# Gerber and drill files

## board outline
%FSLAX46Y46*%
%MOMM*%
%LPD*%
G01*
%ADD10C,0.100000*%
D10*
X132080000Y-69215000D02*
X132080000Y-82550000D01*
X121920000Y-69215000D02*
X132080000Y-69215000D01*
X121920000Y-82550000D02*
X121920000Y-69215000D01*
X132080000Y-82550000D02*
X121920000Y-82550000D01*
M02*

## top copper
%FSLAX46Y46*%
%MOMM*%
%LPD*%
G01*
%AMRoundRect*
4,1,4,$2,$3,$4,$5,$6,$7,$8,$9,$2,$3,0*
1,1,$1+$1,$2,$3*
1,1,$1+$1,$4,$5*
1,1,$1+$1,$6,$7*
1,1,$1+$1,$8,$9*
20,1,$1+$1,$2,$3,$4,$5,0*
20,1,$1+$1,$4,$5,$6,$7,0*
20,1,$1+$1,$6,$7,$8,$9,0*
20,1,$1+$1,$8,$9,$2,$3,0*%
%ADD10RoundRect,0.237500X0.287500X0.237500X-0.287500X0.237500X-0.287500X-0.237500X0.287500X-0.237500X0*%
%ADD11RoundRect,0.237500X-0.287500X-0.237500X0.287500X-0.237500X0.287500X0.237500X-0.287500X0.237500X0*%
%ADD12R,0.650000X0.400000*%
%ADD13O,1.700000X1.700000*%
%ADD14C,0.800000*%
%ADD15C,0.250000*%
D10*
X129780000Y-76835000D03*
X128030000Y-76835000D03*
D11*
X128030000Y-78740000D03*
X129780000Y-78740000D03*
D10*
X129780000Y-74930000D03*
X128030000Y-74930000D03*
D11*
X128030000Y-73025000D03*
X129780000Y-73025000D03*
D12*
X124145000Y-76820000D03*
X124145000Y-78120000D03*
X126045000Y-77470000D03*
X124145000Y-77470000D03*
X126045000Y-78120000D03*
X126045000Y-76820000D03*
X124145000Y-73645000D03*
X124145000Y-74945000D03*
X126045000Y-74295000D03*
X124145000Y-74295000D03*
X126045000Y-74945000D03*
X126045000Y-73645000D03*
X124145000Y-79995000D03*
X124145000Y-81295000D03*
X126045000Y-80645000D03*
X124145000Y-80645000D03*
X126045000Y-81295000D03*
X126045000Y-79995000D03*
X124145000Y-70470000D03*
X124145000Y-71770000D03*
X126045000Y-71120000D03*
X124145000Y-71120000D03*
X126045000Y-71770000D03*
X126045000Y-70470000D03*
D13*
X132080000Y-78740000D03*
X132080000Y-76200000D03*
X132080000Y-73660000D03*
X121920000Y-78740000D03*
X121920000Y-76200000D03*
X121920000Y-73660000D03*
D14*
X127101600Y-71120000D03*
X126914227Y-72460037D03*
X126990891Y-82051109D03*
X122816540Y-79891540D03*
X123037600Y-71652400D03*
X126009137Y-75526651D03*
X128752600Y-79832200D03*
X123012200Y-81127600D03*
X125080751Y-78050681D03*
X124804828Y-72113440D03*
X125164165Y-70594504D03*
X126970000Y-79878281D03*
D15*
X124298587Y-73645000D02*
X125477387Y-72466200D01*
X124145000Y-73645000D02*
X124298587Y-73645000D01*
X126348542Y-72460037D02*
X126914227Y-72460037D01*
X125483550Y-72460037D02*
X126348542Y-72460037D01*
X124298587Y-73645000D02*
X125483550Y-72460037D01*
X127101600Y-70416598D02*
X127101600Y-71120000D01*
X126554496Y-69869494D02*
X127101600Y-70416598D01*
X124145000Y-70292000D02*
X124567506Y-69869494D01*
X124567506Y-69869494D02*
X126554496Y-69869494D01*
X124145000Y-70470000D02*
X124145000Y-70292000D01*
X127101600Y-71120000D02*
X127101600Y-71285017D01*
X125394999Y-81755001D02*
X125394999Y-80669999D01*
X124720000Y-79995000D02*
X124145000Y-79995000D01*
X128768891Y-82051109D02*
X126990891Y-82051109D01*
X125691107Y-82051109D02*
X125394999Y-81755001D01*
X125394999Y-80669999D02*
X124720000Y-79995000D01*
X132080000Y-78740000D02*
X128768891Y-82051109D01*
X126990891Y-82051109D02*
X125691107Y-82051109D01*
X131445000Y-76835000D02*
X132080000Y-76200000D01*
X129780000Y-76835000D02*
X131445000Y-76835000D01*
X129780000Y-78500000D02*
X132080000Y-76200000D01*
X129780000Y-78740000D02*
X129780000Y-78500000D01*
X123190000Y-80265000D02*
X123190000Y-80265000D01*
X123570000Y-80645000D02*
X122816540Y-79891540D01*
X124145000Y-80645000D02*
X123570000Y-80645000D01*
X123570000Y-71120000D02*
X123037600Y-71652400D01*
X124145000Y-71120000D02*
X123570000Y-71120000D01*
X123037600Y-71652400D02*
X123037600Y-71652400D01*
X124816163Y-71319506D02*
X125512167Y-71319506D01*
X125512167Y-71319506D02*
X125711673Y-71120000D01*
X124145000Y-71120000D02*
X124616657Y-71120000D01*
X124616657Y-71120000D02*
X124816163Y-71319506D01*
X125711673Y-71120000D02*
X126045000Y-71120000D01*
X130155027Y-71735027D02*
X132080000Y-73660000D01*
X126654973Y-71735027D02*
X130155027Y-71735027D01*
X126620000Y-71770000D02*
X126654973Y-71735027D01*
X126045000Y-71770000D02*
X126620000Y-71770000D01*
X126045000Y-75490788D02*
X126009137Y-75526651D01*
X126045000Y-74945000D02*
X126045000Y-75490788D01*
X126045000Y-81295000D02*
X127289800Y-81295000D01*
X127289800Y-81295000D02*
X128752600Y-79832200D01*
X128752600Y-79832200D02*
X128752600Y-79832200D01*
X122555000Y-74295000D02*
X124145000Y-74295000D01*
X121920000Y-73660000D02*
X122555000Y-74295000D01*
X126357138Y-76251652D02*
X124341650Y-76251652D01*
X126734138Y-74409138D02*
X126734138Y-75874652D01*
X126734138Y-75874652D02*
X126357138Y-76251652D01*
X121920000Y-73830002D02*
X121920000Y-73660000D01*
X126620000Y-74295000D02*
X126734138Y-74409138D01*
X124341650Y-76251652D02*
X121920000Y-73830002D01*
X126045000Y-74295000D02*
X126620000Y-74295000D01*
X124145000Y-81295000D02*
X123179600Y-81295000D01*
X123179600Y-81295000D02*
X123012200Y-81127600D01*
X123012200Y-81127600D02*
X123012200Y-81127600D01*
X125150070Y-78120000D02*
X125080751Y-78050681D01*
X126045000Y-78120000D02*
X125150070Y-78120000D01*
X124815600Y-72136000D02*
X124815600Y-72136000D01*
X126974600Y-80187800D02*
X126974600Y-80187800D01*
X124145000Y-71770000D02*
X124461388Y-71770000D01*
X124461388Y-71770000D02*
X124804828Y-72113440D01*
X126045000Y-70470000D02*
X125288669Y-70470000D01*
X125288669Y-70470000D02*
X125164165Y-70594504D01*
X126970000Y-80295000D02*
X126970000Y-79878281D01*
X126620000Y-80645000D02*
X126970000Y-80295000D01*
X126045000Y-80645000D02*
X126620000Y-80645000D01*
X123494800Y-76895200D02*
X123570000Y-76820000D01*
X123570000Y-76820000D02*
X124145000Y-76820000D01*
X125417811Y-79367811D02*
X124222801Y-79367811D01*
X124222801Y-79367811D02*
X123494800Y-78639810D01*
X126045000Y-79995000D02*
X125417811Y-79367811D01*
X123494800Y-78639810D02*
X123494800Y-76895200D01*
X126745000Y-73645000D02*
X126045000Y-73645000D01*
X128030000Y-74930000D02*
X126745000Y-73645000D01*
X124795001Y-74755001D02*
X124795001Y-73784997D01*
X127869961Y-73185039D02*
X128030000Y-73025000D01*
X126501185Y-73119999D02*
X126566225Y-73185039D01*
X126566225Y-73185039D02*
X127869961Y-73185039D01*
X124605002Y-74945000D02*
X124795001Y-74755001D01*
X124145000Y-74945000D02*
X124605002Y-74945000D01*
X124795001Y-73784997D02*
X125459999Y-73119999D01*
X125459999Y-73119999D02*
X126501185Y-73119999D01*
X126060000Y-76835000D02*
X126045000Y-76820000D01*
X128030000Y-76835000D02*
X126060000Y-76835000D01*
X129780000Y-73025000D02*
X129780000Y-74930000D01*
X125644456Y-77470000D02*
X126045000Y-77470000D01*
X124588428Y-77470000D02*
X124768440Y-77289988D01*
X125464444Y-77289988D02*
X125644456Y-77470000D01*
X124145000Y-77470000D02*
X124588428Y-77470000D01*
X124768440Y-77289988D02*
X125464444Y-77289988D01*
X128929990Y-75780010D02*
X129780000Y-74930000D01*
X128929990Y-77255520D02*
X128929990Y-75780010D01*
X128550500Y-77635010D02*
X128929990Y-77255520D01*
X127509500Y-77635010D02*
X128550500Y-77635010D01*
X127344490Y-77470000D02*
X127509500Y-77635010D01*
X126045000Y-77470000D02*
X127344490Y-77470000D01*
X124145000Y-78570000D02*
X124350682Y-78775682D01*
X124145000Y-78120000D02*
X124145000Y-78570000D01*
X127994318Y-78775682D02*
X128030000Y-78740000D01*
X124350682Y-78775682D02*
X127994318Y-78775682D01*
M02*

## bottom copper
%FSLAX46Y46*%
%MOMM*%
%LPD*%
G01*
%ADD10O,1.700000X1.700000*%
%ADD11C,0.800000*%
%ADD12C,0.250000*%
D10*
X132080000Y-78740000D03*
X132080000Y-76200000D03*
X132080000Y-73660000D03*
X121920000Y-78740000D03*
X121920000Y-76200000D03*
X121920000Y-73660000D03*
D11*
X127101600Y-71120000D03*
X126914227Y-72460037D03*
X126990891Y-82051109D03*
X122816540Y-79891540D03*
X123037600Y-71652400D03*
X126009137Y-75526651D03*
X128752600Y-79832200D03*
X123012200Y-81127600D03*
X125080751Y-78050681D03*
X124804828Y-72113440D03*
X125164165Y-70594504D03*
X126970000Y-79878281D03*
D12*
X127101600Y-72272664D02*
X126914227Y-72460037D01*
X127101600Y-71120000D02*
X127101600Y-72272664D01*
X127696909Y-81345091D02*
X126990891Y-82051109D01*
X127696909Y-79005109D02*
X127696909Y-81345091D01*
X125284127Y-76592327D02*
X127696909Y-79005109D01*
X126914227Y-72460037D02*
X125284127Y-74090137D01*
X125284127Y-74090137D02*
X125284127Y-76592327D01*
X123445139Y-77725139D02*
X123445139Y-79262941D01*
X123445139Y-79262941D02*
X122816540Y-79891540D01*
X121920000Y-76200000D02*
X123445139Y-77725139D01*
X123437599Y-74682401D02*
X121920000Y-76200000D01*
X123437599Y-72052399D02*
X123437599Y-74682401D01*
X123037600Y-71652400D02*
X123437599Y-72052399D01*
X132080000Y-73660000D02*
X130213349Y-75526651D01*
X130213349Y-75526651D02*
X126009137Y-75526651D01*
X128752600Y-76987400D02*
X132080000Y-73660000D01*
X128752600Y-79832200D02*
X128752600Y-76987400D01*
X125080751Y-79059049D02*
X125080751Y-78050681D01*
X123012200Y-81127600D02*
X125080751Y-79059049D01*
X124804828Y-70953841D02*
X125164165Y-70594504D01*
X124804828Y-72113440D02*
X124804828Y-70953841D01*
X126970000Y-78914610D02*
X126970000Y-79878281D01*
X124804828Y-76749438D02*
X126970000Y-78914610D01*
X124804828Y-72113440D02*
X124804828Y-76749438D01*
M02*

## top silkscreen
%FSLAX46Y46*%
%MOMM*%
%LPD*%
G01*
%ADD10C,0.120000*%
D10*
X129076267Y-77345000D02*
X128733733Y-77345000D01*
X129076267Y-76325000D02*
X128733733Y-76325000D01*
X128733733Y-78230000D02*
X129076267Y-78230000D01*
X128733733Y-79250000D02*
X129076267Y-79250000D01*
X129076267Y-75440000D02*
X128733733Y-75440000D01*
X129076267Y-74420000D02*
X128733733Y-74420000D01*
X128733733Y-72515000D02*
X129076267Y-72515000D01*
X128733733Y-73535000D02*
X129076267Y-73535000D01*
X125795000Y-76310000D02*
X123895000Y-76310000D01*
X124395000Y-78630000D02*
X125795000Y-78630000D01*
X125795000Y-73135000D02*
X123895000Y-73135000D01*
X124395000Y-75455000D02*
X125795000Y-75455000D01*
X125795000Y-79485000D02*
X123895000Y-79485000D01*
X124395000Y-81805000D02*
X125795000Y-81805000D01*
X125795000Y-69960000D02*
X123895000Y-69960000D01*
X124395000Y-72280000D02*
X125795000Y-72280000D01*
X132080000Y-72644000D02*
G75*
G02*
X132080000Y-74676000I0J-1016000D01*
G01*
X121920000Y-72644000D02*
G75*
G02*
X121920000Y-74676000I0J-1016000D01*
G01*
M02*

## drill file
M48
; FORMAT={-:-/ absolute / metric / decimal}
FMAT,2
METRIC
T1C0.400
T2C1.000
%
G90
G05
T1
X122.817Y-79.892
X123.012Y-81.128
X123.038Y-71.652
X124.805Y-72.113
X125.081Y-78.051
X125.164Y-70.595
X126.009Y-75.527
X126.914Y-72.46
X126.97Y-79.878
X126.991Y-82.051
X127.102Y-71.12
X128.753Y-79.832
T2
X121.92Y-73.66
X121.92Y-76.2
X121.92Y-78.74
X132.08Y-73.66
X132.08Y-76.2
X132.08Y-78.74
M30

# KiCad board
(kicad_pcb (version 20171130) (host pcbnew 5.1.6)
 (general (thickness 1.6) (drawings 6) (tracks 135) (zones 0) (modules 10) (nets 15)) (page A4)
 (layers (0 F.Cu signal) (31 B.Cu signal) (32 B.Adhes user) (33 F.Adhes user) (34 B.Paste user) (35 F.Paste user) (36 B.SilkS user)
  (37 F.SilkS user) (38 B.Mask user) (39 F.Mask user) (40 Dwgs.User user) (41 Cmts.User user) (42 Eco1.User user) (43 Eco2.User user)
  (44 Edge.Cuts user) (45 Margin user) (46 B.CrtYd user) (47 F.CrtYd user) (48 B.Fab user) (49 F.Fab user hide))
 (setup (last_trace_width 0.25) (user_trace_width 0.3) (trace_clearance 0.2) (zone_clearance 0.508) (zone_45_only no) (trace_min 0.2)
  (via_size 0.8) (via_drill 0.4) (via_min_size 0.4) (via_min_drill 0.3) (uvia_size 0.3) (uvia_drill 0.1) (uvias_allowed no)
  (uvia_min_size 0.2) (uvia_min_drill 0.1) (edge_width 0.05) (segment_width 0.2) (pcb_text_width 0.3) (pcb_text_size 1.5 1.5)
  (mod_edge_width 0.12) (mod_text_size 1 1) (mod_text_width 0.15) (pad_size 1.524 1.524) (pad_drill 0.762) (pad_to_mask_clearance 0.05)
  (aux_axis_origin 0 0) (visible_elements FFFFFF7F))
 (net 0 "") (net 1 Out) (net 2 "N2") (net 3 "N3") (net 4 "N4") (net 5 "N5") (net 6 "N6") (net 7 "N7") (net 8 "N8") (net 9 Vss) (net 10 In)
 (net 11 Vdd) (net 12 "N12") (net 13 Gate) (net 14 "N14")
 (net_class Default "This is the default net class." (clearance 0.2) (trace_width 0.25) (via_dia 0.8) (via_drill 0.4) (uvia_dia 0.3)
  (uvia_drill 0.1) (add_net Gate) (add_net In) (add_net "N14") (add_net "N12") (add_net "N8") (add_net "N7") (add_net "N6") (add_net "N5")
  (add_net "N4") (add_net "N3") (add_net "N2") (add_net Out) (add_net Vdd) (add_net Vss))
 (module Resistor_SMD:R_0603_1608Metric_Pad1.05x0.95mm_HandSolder (layer F.Cu) (at 128.905 76.835 180)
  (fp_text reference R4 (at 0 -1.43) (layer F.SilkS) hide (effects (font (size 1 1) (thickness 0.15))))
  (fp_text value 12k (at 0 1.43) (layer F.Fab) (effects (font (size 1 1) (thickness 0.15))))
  (fp_line (start -0.171267 -0.51) (end 0.171267 -0.51) (layer F.SilkS) (width 0.12))
  (fp_line (start -0.171267 0.51) (end 0.171267 0.51) (layer F.SilkS) (width 0.12))
  (pad 1 smd roundrect (at -0.875 0 180) (size 1.05 0.95) (layers F.Cu F.Paste F.Mask) (roundrect_rratio 0.25) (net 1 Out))
  (pad 2 smd roundrect (at 0.875 0 180) (size 1.05 0.95) (layers F.Cu F.Paste F.Mask) (roundrect_rratio 0.25) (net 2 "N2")))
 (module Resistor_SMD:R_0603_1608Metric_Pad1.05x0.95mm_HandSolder (layer F.Cu) (at 128.905 78.74)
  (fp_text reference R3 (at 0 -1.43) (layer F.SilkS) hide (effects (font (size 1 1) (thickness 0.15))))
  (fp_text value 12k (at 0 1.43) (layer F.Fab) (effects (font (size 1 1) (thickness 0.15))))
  (fp_line (start -0.171267 -0.51) (end 0.171267 -0.51) (layer F.SilkS) (width 0.12))
  (fp_line (start -0.171267 0.51) (end 0.171267 0.51) (layer F.SilkS) (width 0.12))
  (pad 1 smd roundrect (at -0.875 0) (size 1.05 0.95) (layers F.Cu F.Paste F.Mask) (roundrect_rratio 0.25) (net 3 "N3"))
  (pad 2 smd roundrect (at 0.875 0) (size 1.05 0.95) (layers F.Cu F.Paste F.Mask) (roundrect_rratio 0.25) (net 1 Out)))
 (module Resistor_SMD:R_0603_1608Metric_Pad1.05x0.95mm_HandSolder (layer F.Cu) (at 128.905 74.93 180)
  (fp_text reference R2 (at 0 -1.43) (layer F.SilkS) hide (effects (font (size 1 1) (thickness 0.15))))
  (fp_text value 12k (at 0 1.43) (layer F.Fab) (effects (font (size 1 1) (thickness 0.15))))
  (fp_line (start -0.171267 -0.51) (end 0.171267 -0.51) (layer F.SilkS) (width 0.12))
  (fp_line (start -0.171267 0.51) (end 0.171267 0.51) (layer F.SilkS) (width 0.12))
  (pad 1 smd roundrect (at -0.875 0 180) (size 1.05 0.95) (layers F.Cu F.Paste F.Mask) (roundrect_rratio 0.25) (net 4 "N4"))
  (pad 2 smd roundrect (at 0.875 0 180) (size 1.05 0.95) (layers F.Cu F.Paste F.Mask) (roundrect_rratio 0.25) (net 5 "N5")))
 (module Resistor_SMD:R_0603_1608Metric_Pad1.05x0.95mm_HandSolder (layer F.Cu) (at 128.905 73.025)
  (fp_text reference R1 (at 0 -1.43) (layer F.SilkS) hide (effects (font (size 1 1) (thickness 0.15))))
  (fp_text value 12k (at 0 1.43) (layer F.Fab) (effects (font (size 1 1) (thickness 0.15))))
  (fp_line (start -0.171267 -0.51) (end 0.171267 -0.51) (layer F.SilkS) (width 0.12))
  (fp_line (start -0.171267 0.51) (end 0.171267 0.51) (layer F.SilkS) (width 0.12))
  (pad 1 smd roundrect (at -0.875 0) (size 1.05 0.95) (layers F.Cu F.Paste F.Mask) (roundrect_rratio 0.25) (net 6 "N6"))
  (pad 2 smd roundrect (at 0.875 0) (size 1.05 0.95) (layers F.Cu F.Paste F.Mask) (roundrect_rratio 0.25) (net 4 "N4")))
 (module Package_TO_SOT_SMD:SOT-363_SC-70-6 (layer F.Cu) (at 125.095 77.47)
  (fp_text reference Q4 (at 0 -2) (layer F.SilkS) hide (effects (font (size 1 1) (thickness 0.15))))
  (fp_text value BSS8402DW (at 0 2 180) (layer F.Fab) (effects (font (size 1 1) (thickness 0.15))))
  (fp_line (start 0.7 -1.16) (end -1.2 -1.16) (layer F.SilkS) (width 0.12))
  (fp_line (start -0.7 1.16) (end 0.7 1.16) (layer F.SilkS) (width 0.12))
  (pad 1 smd rect (at -0.95 -0.65) (size 0.65 0.4) (layers F.Cu F.Paste F.Mask) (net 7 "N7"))
  (pad 3 smd rect (at -0.95 0.65) (size 0.65 0.4) (layers F.Cu F.Paste F.Mask) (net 3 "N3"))
  (pad 5 smd rect (at 0.95 0) (size 0.65 0.4) (layers F.Cu F.Paste F.Mask) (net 4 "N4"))
  (pad 2 smd rect (at -0.95 0) (size 0.65 0.4) (layers F.Cu F.Paste F.Mask) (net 4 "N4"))
  (pad 4 smd rect (at 0.95 0.65) (size 0.65 0.4) (layers F.Cu F.Paste F.Mask) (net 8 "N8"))
  (pad 6 smd rect (at 0.95 -0.65) (size 0.65 0.4) (layers F.Cu F.Paste F.Mask) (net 2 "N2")))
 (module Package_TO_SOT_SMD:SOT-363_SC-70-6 (layer F.Cu) (at 125.095 74.295)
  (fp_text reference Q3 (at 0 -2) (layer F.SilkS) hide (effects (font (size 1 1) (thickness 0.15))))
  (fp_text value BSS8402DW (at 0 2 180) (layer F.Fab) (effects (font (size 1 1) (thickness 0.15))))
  (fp_line (start 0.7 -1.16) (end -1.2 -1.16) (layer F.SilkS) (width 0.12))
  (fp_line (start -0.7 1.16) (end 0.7 1.16) (layer F.SilkS) (width 0.12))
  (pad 1 smd rect (at -0.95 -0.65) (size 0.65 0.4) (layers F.Cu F.Paste F.Mask) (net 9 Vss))
  (pad 3 smd rect (at -0.95 0.65) (size 0.65 0.4) (layers F.Cu F.Paste F.Mask) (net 6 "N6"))
  (pad 5 smd rect (at 0.95 0) (size 0.65 0.4) (layers F.Cu F.Paste F.Mask) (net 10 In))
  (pad 2 smd rect (at -0.95 0) (size 0.65 0.4) (layers F.Cu F.Paste F.Mask) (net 10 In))
  (pad 4 smd rect (at 0.95 0.65) (size 0.65 0.4) (layers F.Cu F.Paste F.Mask) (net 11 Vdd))
  (pad 6 smd rect (at 0.95 -0.65) (size 0.65 0.4) (layers F.Cu F.Paste F.Mask) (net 5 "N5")))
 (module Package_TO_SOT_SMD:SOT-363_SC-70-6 (layer F.Cu) (at 125.095 80.645)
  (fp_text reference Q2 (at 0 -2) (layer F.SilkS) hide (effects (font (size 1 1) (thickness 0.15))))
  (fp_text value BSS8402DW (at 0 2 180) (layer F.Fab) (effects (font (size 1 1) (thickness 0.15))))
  (fp_line (start 0.7 -1.16) (end -1.2 -1.16) (layer F.SilkS) (width 0.12))
  (fp_line (start -0.7 1.16) (end 0.7 1.16) (layer F.SilkS) (width 0.12))
  (pad 1 smd rect (at -0.95 -0.65) (size 0.65 0.4) (layers F.Cu F.Paste F.Mask) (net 9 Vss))
  (pad 3 smd rect (at -0.95 0.65) (size 0.65 0.4) (layers F.Cu F.Paste F.Mask) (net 8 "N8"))
  (pad 5 smd rect (at 0.95 0) (size 0.65 0.4) (layers F.Cu F.Paste F.Mask) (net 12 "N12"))
  (pad 2 smd rect (at -0.95 0) (size 0.65 0.4) (layers F.Cu F.Paste F.Mask) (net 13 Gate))
  (pad 4 smd rect (at 0.95 0.65) (size 0.65 0.4) (layers F.Cu F.Paste F.Mask) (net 11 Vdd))
  (pad 6 smd rect (at 0.95 -0.65) (size 0.65 0.4) (layers F.Cu F.Paste F.Mask) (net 7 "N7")))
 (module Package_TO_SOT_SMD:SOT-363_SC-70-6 (layer F.Cu) (at 125.095 71.12)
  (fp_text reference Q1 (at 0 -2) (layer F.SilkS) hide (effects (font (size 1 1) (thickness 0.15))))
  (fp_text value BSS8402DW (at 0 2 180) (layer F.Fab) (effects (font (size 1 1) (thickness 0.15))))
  (fp_line (start 0.7 -1.16) (end -1.2 -1.16) (layer F.SilkS) (width 0.12))
  (fp_line (start -0.7 1.16) (end 0.7 1.16) (layer F.SilkS) (width 0.12))
  (pad 1 smd rect (at -0.95 -0.65) (size 0.65 0.4) (layers F.Cu F.Paste F.Mask) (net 9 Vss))
  (pad 3 smd rect (at -0.95 0.65) (size 0.65 0.4) (layers F.Cu F.Paste F.Mask) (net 12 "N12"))
  (pad 5 smd rect (at 0.95 0) (size 0.65 0.4) (layers F.Cu F.Paste F.Mask) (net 13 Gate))
  (pad 2 smd rect (at -0.95 0) (size 0.65 0.4) (layers F.Cu F.Paste F.Mask) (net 13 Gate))
  (pad 4 smd rect (at 0.95 0.65) (size 0.65 0.4) (layers F.Cu F.Paste F.Mask) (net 11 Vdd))
  (pad 6 smd rect (at 0.95 -0.65) (size 0.65 0.4) (layers F.Cu F.Paste F.Mask) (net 12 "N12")))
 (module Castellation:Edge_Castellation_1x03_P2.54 (layer F.Cu) (at 132.08 73.66)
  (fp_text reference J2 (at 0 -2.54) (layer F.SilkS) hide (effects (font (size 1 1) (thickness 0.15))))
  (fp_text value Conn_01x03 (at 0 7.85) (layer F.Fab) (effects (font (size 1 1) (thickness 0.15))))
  (fp_arc (start 0 0) (end 0 1.016) (angle -180) (layer F.SilkS) (width 0.12))
  (pad 3 thru_hole oval (at 0 5.08) (size 1.7 1.7) (drill 1) (layers *.Cu *.Mask) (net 9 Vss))
  (pad 2 thru_hole oval (at 0 2.54) (size 1.7 1.7) (drill 1) (layers *.Cu *.Mask) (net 1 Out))
  (pad 1 thru_hole oval (at 0 0) (size 1.7 1.7) (drill 1) (layers *.Cu *.Mask) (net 11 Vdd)))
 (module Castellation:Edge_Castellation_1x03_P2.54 (layer F.Cu) (at 121.92 73.66)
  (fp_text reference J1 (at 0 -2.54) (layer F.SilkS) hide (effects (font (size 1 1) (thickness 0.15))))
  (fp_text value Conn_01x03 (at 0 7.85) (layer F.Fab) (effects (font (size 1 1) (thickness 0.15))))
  (fp_arc (start 0 0) (end 0 1.016) (angle -180) (layer F.SilkS) (width 0.12))
  (pad 3 thru_hole oval (at 0 5.08) (size 1.7 1.7) (drill 1) (layers *.Cu *.Mask) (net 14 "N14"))
  (pad 2 thru_hole oval (at 0 2.54) (size 1.7 1.7) (drill 1) (layers *.Cu *.Mask) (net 13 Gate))
  (pad 1 thru_hole oval (at 0 0) (size 1.7 1.7) (drill 1) (layers *.Cu *.Mask) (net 10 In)))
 (gr_line (start 132.08 69.215) (end 132.08 82.55) (layer Edge.Cuts) (width 0.1))
 (gr_line (start 121.92 69.215) (end 132.08 69.215) (layer Edge.Cuts) (width 0.1))
 (gr_line (start 121.92 82.55) (end 121.92 69.215) (layer Edge.Cuts) (width 0.1))
 (gr_line (start 132.08 82.55) (end 121.92 82.55) (layer Edge.Cuts) (width 0.1))
 (via (at 127.1016 71.12) (size 0.8) (drill 0.4) (layers F.Cu B.Cu) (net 9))
 (segment (start 124.298587 73.645) (end 125.477387 72.4662) (width 0.25) (layer F.Cu) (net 9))
 (segment (start 124.145 73.645) (end 124.298587 73.645) (width 0.25) (layer F.Cu) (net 9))
 (segment (start 126.348542 72.460037) (end 126.914227 72.460037) (width 0.25) (layer F.Cu) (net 9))
 (segment (start 125.48355 72.460037) (end 126.348542 72.460037) (width 0.25) (layer F.Cu) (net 9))
 (via (at 126.914227 72.460037) (size 0.8) (drill 0.4) (layers F.Cu B.Cu) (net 9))
 (segment (start 124.298587 73.645) (end 125.48355 72.460037) (width 0.25) (layer F.Cu) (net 9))
 (segment (start 127.1016 70.416598) (end 127.1016 71.12) (width 0.25) (layer F.Cu) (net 9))
 (segment (start 126.554496 69.869494) (end 127.1016 70.416598) (width 0.25) (layer F.Cu) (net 9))
 (segment (start 124.145 70.292) (end 124.567506 69.869494) (width 0.25) (layer F.Cu) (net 9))
 (segment (start 124.567506 69.869494) (end 126.554496 69.869494) (width 0.25) (layer F.Cu) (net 9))
 (segment (start 124.145 70.47) (end 124.145 70.292) (width 0.25) (layer F.Cu) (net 9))
 (segment (start 127.1016 71.12) (end 127.1016 71.285017) (width 0.25) (layer F.Cu) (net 9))
 (segment (start 127.1016 72.272664) (end 126.914227 72.460037) (width 0.25) (layer B.Cu) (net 9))
 (segment (start 127.1016 71.12) (end 127.1016 72.272664) (width 0.25) (layer B.Cu) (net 9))
 (segment (start 125.394999 81.755001) (end 125.394999 80.669999) (width 0.25) (layer F.Cu) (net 9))
 (segment (start 124.72 79.995) (end 124.145 79.995) (width 0.25) (layer F.Cu) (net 9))
 (segment (start 128.768891 82.051109) (end 126.990891 82.051109) (width 0.25) (layer F.Cu) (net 9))
 (segment (start 125.691107 82.051109) (end 125.394999 81.755001) (width 0.25) (layer F.Cu) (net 9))
 (segment (start 125.394999 80.669999) (end 124.72 79.995) (width 0.25) (layer F.Cu) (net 9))
 (segment (start 132.08 78.74) (end 128.768891 82.051109) (width 0.25) (layer F.Cu) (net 9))
 (segment (start 126.990891 82.051109) (end 125.691107 82.051109) (width 0.25) (layer F.Cu) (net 9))
 (via (at 126.990891 82.051109) (size 0.8) (drill 0.4) (layers F.Cu B.Cu) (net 9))
 (segment (start 127.696909 81.345091) (end 126.990891 82.051109) (width 0.25) (layer B.Cu) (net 9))
 (segment (start 127.696909 79.005109) (end 127.696909 81.345091) (width 0.25) (layer B.Cu) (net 9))
 (segment (start 125.284127 76.592327) (end 127.696909 79.005109) (width 0.25) (layer B.Cu) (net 9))
 (segment (start 126.914227 72.460037) (end 125.284127 74.090137) (width 0.25) (layer B.Cu) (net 9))
 (segment (start 125.284127 74.090137) (end 125.284127 76.592327) (width 0.25) (layer B.Cu) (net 9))
 (segment (start 131.445 76.835) (end 132.08 76.2) (width 0.25) (layer F.Cu) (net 1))
 (segment (start 129.78 76.835) (end 131.445 76.835) (width 0.25) (layer F.Cu) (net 1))
 (segment (start 129.78 78.5) (end 132.08 76.2) (width 0.25) (layer F.Cu) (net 1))
 (segment (start 129.78 78.74) (end 129.78 78.5) (width 0.25) (layer F.Cu) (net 1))
 (segment (start 123.19 80.265) (end 123.19 80.265) (width 0.25) (layer F.Cu) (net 13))
 (segment (start 123.445139 77.725139) (end 123.445139 79.262941) (width 0.25) (layer B.Cu) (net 13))
 (segment (start 123.57 80.645) (end 122.81654 79.89154) (width 0.25) (layer F.Cu) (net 13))
 (segment (start 124.145 80.645) (end 123.57 80.645) (width 0.25) (layer F.Cu) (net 13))
 (segment (start 123.445139 79.262941) (end 122.81654 79.89154) (width 0.25) (layer B.Cu) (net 13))
 (via (at 122.81654 79.89154) (size 0.8) (drill 0.4) (layers F.Cu B.Cu) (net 13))
 (segment (start 121.92 76.2) (end 123.445139 77.725139) (width 0.25) (layer B.Cu) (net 13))
 (segment (start 123.57 71.12) (end 123.0376 71.6524) (width 0.25) (layer F.Cu) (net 13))
 (segment (start 124.145 71.12) (end 123.57 71.12) (width 0.25) (layer F.Cu) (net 13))
 (segment (start 123.0376 71.6524) (end 123.0376 71.6524) (width 0.25) (layer F.Cu) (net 13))
 (via (at 123.0376 71.6524) (size 0.8) (drill 0.4) (layers F.Cu B.Cu) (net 13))
 (segment (start 123.437599 74.682401) (end 121.92 76.2) (width 0.25) (layer B.Cu) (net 13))
 (segment (start 123.437599 72.052399) (end 123.437599 74.682401) (width 0.25) (layer B.Cu) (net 13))
 (segment (start 123.0376 71.6524) (end 123.437599 72.052399) (width 0.25) (layer B.Cu) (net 13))
 (segment (start 124.816163 71.319506) (end 125.512167 71.319506) (width 0.25) (layer F.Cu) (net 13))
 (segment (start 125.512167 71.319506) (end 125.711673 71.12) (width 0.25) (layer F.Cu) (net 13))
 (segment (start 124.145 71.12) (end 124.616657 71.12) (width 0.25) (layer F.Cu) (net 13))
 (segment (start 124.616657 71.12) (end 124.816163 71.319506) (width 0.25) (layer F.Cu) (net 13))
 (segment (start 125.711673 71.12) (end 126.045 71.12) (width 0.25) (layer F.Cu) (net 13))
 (segment (start 130.155027 71.735027) (end 132.08 73.66) (width 0.25) (layer F.Cu) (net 11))
 (segment (start 126.654973 71.735027) (end 130.155027 71.735027) (width 0.25) (layer F.Cu) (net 11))
 (segment (start 126.62 71.77) (end 126.654973 71.735027) (width 0.25) (layer F.Cu) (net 11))
 (segment (start 126.045 71.77) (end 126.62 71.77) (width 0.25) (layer F.Cu) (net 11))
 (via (at 126.009137 75.526651) (size 0.8) (drill 0.4) (layers F.Cu B.Cu) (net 11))
 (segment (start 132.08 73.66) (end 130.213349 75.526651) (width 0.25) (layer B.Cu) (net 11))
 (segment (start 130.213349 75.526651) (end 126.009137 75.526651) (width 0.25) (layer B.Cu) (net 11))
 (segment (start 126.045 75.490788) (end 126.009137 75.526651) (width 0.25) (layer F.Cu) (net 11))
 (segment (start 126.045 74.945) (end 126.045 75.490788) (width 0.25) (layer F.Cu) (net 11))
 (segment (start 126.045 81.295) (end 127.2898 81.295) (width 0.25) (layer F.Cu) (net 11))
 (segment (start 127.2898 81.295) (end 128.7526 79.8322) (width 0.25) (layer F.Cu) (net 11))
 (segment (start 128.7526 79.8322) (end 128.7526 79.8322) (width 0.25) (layer F.Cu) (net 11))
 (via (at 128.7526 79.8322) (size 0.8) (drill 0.4) (layers F.Cu B.Cu) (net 11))
 (segment (start 128.7526 76.9874) (end 132.08 73.66) (width 0.25) (layer B.Cu) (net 11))
 (segment (start 128.7526 79.8322) (end 128.7526 76.9874) (width 0.25) (layer B.Cu) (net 11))
 (segment (start 122.555 74.295) (end 124.145 74.295) (width 0.25) (layer F.Cu) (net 10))
 (segment (start 121.92 73.66) (end 122.555 74.295) (width 0.25) (layer F.Cu) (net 10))
 (segment (start 126.357138 76.251652) (end 124.34165 76.251652) (width 0.25) (layer F.Cu) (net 10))
 (segment (start 126.734138 74.409138) (end 126.734138 75.874652) (width 0.25) (layer F.Cu) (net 10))
 (segment (start 126.734138 75.874652) (end 126.357138 76.251652) (width 0.25) (layer F.Cu) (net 10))
 (segment (start 121.92 73.830002) (end 121.92 73.66) (width 0.25) (layer F.Cu) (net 10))
 (segment (start 126.62 74.295) (end 126.734138 74.409138) (width 0.25) (layer F.Cu) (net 10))
 (segment (start 124.34165 76.251652) (end 121.92 73.830002) (width 0.25) (layer F.Cu) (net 10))
 (segment (start 126.045 74.295) (end 126.62 74.295) (width 0.25) (layer F.Cu) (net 10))
 (segment (start 124.145 81.295) (end 123.1796 81.295) (width 0.25) (layer F.Cu) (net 8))
 (segment (start 123.1796 81.295) (end 123.0122 81.1276) (width 0.25) (layer F.Cu) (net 8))
 (segment (start 123.0122 81.1276) (end 123.0122 81.1276) (width 0.25) (layer F.Cu) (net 8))
 (via (at 123.0122 81.1276) (size 0.8) (drill 0.4) (layers F.Cu B.Cu) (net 8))
 (segment (start 125.15007 78.12) (end 125.080751 78.050681) (width 0.25) (layer F.Cu) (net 8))
 (via (at 125.080751 78.050681) (size 0.8) (drill 0.4) (layers F.Cu B.Cu) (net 8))
 (segment (start 125.080751 79.059049) (end 125.080751 78.050681) (width 0.25) (layer B.Cu) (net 8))
 (segment (start 123.0122 81.1276) (end 125.080751 79.059049) (width 0.25) (layer B.Cu) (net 8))
 (segment (start 126.045 78.12) (end 125.15007 78.12) (width 0.25) (layer F.Cu) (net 8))
 (segment (start 124.8156 72.136) (end 124.8156 72.136) (width 0.25) (layer F.Cu) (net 12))
 (segment (start 126.9746 80.1878) (end 126.9746 80.1878) (width 0.25) (layer F.Cu) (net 12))
 (via (at 124.804828 72.11344) (size 0.8) (drill 0.4) (layers F.Cu B.Cu) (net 12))
 (segment (start 124.145 71.77) (end 124.461388 71.77) (width 0.25) (layer F.Cu) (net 12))
 (segment (start 124.461388 71.77) (end 124.804828 72.11344) (width 0.25) (layer F.Cu) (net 12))
 (segment (start 126.045 70.47) (end 125.288669 70.47) (width 0.25) (layer F.Cu) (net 12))
 (segment (start 124.804828 70.953841) (end 125.164165 70.594504) (width 0.25) (layer B.Cu) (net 12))
 (segment (start 124.804828 72.11344) (end 124.804828 70.953841) (width 0.25) (layer B.Cu) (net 12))
 (segment (start 125.288669 70.47) (end 125.164165 70.594504) (width 0.25) (layer F.Cu) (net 12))
 (via (at 125.164165 70.594504) (size 0.8) (drill 0.4) (layers F.Cu B.Cu) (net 12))
 (segment (start 126.97 78.91461) (end 126.97 79.878281) (width 0.25) (layer B.Cu) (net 12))
 (via (at 126.97 79.878281) (size 0.8) (drill 0.4) (layers F.Cu B.Cu) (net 12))
 (segment (start 126.97 80.295) (end 126.97 79.878281) (width 0.25) (layer F.Cu) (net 12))
 (segment (start 124.804828 76.749438) (end 126.97 78.91461) (width 0.25) (layer B.Cu) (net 12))
 (segment (start 124.804828 72.11344) (end 124.804828 76.749438) (width 0.25) (layer B.Cu) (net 12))
 (segment (start 126.62 80.645) (end 126.97 80.295) (width 0.25) (layer F.Cu) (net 12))
 (segment (start 126.045 80.645) (end 126.62 80.645) (width 0.25) (layer F.Cu) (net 12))
 (segment (start 123.4948 76.8952) (end 123.57 76.82) (width 0.25) (layer F.Cu) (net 7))
 (segment (start 123.57 76.82) (end 124.145 76.82) (width 0.25) (layer F.Cu) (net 7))
 (segment (start 125.417811 79.367811) (end 124.222801 79.367811) (width 0.25) (layer F.Cu) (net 7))
 (segment (start 124.222801 79.367811) (end 123.4948 78.63981) (width 0.25) (layer F.Cu) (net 7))
 (segment (start 126.045 79.995) (end 125.417811 79.367811) (width 0.25) (layer F.Cu) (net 7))
 (segment (start 123.4948 78.63981) (end 123.4948 76.8952) (width 0.25) (layer F.Cu) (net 7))
 (segment (start 126.745 73.645) (end 126.045 73.645) (width 0.25) (layer F.Cu) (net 5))
 (segment (start 128.03 74.93) (end 126.745 73.645) (width 0.25) (layer F.Cu) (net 5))
 (segment (start 124.795001 74.755001) (end 124.795001 73.784997) (width 0.25) (layer F.Cu) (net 6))
 (segment (start 127.869961 73.185039) (end 128.03 73.025) (width 0.25) (layer F.Cu) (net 6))
 (segment (start 126.501185 73.119999) (end 126.566225 73.185039) (width 0.25) (layer F.Cu) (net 6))
 (segment (start 126.566225 73.185039) (end 127.869961 73.185039) (width 0.25) (layer F.Cu) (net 6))
 (segment (start 124.605002 74.945) (end 124.795001 74.755001) (width 0.25) (layer F.Cu) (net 6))
 (segment (start 124.145 74.945) (end 124.605002 74.945) (width 0.25) (layer F.Cu) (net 6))
 (segment (start 124.795001 73.784997) (end 125.459999 73.119999) (width 0.25) (layer F.Cu) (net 6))
 (segment (start 125.459999 73.119999) (end 126.501185 73.119999) (width 0.25) (layer F.Cu) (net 6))
 (segment (start 126.06 76.835) (end 126.045 76.82) (width 0.25) (layer F.Cu) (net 2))
 (segment (start 128.03 76.835) (end 126.06 76.835) (width 0.25) (layer F.Cu) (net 2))
 (segment (start 129.78 73.025) (end 129.78 74.93) (width 0.25) (layer F.Cu) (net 4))
 (segment (start 125.644456 77.47) (end 126.045 77.47) (width 0.25) (layer F.Cu) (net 4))
 (segment (start 124.588428 77.47) (end 124.76844 77.289988) (width 0.25) (layer F.Cu) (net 4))
 (segment (start 125.464444 77.289988) (end 125.644456 77.47) (width 0.25) (layer F.Cu) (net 4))
 (segment (start 124.145 77.47) (end 124.588428 77.47) (width 0.25) (layer F.Cu) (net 4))
 (segment (start 124.76844 77.289988) (end 125.464444 77.289988) (width 0.25) (layer F.Cu) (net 4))
 (segment (start 128.92999 75.78001) (end 129.78 74.93) (width 0.25) (layer F.Cu) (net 4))
 (segment (start 128.92999 77.25552) (end 128.92999 75.78001) (width 0.25) (layer F.Cu) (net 4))
 (segment (start 128.5505 77.63501) (end 128.92999 77.25552) (width 0.25) (layer F.Cu) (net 4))
 (segment (start 127.5095 77.63501) (end 128.5505 77.63501) (width 0.25) (layer F.Cu) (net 4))
 (segment (start 127.34449 77.47) (end 127.5095 77.63501) (width 0.25) (layer F.Cu) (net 4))
 (segment (start 126.045 77.47) (end 127.34449 77.47) (width 0.25) (layer F.Cu) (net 4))
 (segment (start 124.145 78.57) (end 124.350682 78.775682) (width 0.25) (layer F.Cu) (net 3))
 (segment (start 124.145 78.12) (end 124.145 78.57) (width 0.25) (layer F.Cu) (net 3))
 (segment (start 127.994318 78.775682) (end 128.03 78.74) (width 0.25) (layer F.Cu) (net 3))
 (segment (start 124.350682 78.775682) (end 127.994318 78.775682) (width 0.25) (layer F.Cu) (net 3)))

